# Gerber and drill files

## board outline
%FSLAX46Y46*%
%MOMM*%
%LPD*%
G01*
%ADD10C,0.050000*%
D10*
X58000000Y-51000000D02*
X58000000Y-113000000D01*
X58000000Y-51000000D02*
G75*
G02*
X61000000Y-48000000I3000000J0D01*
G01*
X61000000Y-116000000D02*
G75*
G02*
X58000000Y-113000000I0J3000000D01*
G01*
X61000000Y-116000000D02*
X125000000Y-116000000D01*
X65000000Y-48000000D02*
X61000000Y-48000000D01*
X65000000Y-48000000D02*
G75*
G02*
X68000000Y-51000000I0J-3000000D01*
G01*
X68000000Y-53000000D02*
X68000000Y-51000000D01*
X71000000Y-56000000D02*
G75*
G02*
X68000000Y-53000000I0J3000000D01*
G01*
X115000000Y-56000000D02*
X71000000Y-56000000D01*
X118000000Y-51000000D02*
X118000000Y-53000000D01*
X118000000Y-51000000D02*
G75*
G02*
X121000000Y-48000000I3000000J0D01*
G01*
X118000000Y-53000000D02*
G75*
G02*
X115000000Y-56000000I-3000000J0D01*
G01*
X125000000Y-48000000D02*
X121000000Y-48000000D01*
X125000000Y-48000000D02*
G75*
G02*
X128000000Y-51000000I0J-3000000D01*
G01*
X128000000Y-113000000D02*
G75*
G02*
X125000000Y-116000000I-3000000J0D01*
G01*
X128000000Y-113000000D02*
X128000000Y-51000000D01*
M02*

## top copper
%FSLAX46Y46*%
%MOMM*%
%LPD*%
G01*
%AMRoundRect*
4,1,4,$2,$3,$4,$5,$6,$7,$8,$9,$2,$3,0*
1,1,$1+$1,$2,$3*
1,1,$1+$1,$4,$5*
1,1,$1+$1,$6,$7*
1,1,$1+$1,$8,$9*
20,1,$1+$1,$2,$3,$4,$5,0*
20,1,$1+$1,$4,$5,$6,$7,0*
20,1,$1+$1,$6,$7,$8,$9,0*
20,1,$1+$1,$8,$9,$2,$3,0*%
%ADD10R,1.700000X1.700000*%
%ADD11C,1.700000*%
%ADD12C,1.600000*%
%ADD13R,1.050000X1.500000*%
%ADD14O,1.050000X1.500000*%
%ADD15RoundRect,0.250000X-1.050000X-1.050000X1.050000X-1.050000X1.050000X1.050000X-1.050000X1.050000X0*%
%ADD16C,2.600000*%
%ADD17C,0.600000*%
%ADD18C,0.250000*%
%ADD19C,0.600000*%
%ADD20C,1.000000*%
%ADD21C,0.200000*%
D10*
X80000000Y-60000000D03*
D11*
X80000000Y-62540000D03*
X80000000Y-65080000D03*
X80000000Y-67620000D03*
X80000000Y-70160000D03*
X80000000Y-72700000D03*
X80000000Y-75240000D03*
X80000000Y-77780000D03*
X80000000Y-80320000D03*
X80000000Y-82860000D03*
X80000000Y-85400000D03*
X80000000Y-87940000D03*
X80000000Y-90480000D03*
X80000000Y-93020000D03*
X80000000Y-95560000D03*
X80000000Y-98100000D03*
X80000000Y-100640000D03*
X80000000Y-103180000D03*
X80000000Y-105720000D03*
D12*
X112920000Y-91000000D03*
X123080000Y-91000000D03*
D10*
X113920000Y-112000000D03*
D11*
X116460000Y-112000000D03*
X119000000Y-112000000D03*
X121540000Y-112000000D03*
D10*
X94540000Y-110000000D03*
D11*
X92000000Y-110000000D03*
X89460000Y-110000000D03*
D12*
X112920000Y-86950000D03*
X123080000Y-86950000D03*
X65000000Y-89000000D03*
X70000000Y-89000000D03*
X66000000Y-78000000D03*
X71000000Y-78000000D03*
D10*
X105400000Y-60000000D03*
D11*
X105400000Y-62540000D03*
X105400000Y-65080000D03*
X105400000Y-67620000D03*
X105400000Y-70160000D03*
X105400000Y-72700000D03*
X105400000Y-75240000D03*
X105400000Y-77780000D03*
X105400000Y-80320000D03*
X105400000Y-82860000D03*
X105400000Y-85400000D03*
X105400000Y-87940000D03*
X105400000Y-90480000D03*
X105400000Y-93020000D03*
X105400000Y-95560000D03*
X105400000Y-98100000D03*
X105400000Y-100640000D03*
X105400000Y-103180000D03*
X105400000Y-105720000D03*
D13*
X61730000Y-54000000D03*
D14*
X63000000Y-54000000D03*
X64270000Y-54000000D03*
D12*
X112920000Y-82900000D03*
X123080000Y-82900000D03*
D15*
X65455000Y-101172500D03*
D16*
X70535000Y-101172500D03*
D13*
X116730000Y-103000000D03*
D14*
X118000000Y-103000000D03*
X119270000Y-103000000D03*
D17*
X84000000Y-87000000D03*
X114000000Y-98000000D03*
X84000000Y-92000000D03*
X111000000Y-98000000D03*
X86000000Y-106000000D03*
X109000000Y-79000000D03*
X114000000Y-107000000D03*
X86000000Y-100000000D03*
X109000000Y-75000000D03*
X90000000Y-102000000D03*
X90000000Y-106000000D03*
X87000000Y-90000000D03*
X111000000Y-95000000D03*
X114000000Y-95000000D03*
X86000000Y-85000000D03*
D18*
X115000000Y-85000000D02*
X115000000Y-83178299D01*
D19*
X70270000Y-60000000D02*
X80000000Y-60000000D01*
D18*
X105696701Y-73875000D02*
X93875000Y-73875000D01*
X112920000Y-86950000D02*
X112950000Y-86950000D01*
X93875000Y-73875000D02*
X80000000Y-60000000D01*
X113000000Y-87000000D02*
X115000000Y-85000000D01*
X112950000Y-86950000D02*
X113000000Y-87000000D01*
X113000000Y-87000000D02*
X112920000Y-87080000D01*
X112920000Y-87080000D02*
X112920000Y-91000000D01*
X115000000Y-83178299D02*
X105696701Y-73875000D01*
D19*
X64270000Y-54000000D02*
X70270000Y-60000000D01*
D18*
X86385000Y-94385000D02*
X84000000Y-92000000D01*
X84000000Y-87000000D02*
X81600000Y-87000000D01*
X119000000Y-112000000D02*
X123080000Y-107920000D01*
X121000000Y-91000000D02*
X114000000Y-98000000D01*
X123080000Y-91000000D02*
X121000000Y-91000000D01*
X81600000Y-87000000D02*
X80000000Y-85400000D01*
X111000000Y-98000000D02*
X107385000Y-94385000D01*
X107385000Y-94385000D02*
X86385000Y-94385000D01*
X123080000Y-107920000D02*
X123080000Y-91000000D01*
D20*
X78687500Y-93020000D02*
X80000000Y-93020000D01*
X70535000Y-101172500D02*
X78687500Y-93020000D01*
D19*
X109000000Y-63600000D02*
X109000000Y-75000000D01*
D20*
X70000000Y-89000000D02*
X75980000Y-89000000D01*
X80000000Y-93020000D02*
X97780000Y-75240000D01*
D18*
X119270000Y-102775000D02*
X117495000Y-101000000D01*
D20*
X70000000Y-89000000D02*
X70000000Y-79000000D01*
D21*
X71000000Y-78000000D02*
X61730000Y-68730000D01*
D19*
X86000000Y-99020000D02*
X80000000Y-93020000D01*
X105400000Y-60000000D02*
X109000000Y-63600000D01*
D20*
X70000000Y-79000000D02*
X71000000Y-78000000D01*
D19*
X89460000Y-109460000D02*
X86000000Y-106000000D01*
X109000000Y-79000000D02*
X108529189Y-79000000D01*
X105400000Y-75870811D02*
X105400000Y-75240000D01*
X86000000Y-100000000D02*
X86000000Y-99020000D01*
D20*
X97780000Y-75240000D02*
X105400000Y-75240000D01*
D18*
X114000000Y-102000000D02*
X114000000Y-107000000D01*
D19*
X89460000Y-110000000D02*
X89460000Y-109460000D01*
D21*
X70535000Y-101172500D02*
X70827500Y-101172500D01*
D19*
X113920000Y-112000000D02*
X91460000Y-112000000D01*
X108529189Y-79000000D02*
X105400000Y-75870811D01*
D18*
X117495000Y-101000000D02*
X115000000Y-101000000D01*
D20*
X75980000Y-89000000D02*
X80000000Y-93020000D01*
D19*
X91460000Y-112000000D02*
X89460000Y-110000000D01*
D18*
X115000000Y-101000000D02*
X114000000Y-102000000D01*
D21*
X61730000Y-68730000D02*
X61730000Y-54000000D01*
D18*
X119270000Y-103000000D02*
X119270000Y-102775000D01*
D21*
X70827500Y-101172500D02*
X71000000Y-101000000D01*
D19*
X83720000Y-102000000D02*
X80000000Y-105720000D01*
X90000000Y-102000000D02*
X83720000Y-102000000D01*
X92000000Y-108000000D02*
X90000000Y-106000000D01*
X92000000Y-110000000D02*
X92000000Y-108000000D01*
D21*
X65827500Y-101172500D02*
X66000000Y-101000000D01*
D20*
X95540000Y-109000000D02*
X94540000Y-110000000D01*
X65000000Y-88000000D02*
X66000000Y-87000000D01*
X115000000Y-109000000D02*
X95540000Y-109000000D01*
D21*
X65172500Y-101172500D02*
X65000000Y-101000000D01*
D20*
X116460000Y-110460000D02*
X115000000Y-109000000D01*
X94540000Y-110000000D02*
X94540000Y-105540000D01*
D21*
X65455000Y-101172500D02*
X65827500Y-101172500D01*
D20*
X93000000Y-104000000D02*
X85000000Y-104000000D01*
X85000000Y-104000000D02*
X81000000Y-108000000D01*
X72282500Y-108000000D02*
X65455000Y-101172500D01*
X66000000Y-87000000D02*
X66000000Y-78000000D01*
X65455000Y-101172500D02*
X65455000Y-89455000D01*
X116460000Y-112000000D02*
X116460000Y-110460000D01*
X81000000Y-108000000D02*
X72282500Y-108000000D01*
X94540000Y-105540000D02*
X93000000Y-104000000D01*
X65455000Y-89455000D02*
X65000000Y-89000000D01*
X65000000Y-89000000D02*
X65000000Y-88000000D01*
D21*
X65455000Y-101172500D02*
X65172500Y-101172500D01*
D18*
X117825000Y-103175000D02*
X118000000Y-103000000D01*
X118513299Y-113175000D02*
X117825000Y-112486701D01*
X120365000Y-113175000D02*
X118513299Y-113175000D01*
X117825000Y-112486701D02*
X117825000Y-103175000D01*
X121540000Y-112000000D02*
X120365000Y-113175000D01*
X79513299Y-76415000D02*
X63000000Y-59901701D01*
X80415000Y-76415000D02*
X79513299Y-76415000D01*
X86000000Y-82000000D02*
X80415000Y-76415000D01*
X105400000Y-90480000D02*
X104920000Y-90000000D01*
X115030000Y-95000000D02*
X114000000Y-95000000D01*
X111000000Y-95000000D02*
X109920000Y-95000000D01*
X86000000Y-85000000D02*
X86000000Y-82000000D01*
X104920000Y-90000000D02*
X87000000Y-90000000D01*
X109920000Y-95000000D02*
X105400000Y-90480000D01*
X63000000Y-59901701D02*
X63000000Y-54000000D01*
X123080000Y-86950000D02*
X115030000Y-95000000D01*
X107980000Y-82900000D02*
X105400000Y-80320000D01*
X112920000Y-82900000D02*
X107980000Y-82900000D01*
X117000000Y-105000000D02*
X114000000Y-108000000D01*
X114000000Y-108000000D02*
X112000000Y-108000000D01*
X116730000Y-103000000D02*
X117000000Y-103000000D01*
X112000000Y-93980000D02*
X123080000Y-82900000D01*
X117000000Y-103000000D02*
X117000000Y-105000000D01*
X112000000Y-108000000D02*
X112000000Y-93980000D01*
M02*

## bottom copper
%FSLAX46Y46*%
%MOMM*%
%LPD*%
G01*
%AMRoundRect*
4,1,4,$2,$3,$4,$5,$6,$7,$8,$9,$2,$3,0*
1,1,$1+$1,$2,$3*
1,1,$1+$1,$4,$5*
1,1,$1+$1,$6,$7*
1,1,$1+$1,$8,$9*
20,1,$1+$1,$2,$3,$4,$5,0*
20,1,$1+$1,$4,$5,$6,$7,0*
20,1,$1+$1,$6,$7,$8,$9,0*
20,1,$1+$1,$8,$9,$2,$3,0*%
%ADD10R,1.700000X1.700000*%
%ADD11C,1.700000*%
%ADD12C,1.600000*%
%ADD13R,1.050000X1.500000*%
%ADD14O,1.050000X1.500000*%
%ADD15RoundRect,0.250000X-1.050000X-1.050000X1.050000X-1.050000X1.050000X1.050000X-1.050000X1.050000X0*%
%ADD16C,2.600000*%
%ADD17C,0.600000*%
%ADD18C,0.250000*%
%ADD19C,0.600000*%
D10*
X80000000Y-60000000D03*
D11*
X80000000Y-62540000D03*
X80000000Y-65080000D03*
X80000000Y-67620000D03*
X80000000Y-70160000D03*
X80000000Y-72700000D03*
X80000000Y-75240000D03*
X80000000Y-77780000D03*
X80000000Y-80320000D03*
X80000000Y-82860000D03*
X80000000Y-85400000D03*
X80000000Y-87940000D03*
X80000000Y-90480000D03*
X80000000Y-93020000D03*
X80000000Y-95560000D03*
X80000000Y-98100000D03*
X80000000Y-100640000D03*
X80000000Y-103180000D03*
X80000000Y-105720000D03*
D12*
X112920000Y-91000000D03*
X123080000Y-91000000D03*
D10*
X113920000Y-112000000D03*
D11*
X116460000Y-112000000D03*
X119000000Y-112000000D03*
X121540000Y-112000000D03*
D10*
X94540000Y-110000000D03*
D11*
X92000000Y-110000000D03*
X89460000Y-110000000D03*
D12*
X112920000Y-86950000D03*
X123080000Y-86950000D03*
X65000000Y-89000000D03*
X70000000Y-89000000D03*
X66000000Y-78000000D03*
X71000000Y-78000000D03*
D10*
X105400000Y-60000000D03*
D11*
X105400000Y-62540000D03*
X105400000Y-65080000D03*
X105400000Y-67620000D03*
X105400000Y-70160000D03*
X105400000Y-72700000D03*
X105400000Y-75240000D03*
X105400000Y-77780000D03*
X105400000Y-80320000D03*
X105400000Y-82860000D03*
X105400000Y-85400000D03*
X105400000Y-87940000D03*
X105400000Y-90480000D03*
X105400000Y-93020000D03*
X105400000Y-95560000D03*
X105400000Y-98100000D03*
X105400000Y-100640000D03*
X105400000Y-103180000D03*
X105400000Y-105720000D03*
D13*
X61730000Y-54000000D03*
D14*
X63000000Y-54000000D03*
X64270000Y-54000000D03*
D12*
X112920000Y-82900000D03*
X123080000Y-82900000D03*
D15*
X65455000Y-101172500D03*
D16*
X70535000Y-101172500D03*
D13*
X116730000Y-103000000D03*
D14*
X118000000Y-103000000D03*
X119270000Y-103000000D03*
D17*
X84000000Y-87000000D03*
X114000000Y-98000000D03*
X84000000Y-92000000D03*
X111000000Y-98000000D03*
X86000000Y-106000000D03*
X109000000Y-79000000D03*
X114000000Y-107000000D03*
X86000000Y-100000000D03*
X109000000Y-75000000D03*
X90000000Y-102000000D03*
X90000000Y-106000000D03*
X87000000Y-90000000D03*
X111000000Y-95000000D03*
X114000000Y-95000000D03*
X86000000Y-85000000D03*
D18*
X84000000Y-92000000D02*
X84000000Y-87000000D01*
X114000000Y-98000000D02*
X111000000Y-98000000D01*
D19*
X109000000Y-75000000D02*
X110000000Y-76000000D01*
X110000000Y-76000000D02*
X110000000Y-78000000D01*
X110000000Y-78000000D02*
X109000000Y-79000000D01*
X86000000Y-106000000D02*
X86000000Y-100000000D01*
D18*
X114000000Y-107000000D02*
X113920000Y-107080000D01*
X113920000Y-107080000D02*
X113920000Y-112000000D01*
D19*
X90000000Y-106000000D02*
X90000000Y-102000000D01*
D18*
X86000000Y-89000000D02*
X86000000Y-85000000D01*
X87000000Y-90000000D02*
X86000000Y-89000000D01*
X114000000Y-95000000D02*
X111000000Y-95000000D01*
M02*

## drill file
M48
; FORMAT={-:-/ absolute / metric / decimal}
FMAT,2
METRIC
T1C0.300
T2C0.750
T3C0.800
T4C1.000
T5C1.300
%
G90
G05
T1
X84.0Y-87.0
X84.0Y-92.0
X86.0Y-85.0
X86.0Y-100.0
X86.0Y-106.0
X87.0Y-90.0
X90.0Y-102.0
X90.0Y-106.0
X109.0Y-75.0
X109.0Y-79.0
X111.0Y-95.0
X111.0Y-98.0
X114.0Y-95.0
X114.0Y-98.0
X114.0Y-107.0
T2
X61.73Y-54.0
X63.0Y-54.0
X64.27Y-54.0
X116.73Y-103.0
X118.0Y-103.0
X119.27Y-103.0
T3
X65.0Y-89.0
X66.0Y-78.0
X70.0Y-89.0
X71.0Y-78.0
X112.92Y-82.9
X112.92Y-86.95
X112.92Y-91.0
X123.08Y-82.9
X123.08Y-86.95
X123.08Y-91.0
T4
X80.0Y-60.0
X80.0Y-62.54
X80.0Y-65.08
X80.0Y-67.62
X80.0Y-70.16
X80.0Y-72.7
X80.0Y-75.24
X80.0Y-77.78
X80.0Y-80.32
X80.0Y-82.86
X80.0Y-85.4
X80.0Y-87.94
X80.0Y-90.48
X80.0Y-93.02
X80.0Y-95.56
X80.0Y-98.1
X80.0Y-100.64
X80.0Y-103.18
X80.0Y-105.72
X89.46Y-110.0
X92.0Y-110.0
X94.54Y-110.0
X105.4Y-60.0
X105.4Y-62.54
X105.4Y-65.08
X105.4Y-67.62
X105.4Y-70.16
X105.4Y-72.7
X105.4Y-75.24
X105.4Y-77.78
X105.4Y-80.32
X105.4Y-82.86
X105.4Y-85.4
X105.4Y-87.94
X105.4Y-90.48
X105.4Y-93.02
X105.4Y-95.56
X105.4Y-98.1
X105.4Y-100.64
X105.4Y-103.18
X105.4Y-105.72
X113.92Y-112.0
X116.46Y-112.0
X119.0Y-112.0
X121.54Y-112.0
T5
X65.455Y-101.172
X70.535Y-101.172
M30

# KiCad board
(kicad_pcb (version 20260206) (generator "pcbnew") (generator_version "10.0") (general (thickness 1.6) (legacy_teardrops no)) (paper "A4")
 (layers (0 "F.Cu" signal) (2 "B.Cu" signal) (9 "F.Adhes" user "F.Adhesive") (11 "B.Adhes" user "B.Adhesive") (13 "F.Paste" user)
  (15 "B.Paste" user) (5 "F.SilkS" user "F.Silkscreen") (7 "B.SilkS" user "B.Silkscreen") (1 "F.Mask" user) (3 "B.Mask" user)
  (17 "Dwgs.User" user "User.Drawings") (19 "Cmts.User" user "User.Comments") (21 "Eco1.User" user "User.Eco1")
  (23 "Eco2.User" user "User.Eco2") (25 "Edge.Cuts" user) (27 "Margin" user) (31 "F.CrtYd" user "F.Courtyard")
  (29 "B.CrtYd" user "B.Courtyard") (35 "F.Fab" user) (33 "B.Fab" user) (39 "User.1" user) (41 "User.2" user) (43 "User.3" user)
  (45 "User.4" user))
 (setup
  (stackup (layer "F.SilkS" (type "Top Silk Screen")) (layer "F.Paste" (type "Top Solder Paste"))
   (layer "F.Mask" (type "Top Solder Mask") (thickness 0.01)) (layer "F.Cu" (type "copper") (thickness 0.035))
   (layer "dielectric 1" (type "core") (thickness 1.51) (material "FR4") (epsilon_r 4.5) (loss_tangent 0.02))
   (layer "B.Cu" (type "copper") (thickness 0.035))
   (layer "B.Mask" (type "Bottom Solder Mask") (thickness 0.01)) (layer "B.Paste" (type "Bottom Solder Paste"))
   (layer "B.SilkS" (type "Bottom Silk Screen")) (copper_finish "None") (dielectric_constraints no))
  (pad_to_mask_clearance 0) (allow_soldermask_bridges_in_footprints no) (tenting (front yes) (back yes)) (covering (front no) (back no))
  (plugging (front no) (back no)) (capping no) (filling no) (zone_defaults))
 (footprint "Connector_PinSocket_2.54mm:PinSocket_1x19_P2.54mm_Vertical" (layer "F.Cu") (at 80 60)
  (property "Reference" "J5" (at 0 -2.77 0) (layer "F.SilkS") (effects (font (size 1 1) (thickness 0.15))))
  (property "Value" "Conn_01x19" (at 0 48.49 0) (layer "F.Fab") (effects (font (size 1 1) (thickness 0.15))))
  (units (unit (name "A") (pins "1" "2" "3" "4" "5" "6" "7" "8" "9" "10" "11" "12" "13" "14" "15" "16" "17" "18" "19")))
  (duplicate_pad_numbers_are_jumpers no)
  (pad "1" thru_hole rect (at 0 0) (size 1.7 1.7) (drill 1) (layers "*.Cu" "*.Mask") (remove_unused_layers no) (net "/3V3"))
  (pad "2" thru_hole circle (at 0 2.54) (size 1.7 1.7) (drill 1) (layers "*.Cu" "*.Mask") (remove_unused_layers no)
   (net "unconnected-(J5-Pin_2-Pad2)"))
  (pad "3" thru_hole circle (at 0 5.08) (size 1.7 1.7) (drill 1) (layers "*.Cu" "*.Mask") (remove_unused_layers no)
   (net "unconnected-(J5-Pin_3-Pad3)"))
  (pad "4" thru_hole circle (at 0 7.62) (size 1.7 1.7) (drill 1) (layers "*.Cu" "*.Mask") (remove_unused_layers no)
   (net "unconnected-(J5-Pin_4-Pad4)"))
  (pad "5" thru_hole circle (at 0 10.16) (size 1.7 1.7) (drill 1) (layers "*.Cu" "*.Mask") (remove_unused_layers no)
   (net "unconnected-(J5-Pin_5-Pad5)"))
  (pad "6" thru_hole circle (at 0 12.7) (size 1.7 1.7) (drill 1) (layers "*.Cu" "*.Mask") (remove_unused_layers no)
   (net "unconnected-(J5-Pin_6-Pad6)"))
  (pad "7" thru_hole circle (at 0 15.24) (size 1.7 1.7) (drill 1) (layers "*.Cu" "*.Mask") (remove_unused_layers no)
   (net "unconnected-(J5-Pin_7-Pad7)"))
  (pad "8" thru_hole circle (at 0 17.78) (size 1.7 1.7) (drill 1) (layers "*.Cu" "*.Mask") (remove_unused_layers no)
   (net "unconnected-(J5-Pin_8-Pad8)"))
  (pad "9" thru_hole circle (at 0 20.32) (size 1.7 1.7) (drill 1) (layers "*.Cu" "*.Mask") (remove_unused_layers no)
   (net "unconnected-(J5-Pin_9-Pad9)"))
  (pad "10" thru_hole circle (at 0 22.86) (size 1.7 1.7) (drill 1) (layers "*.Cu" "*.Mask") (remove_unused_layers no)
   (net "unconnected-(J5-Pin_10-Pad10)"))
  (pad "11" thru_hole circle (at 0 25.4) (size 1.7 1.7) (drill 1) (layers "*.Cu" "*.Mask") (remove_unused_layers no) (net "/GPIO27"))
  (pad "12" thru_hole circle (at 0 27.94) (size 1.7 1.7) (drill 1) (layers "*.Cu" "*.Mask") (remove_unused_layers no)
   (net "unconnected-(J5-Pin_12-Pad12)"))
  (pad "13" thru_hole circle (at 0 30.48) (size 1.7 1.7) (drill 1) (layers "*.Cu" "*.Mask") (remove_unused_layers no)
   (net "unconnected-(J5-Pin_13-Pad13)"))
  (pad "14" thru_hole circle (at 0 33.02) (size 1.7 1.7) (drill 1) (layers "*.Cu" "*.Mask") (remove_unused_layers no) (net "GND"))
  (pad "15" thru_hole circle (at 0 35.56) (size 1.7 1.7) (drill 1) (layers "*.Cu" "*.Mask") (remove_unused_layers no)
   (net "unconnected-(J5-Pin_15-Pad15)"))
  (pad "16" thru_hole circle (at 0 38.1) (size 1.7 1.7) (drill 1) (layers "*.Cu" "*.Mask") (remove_unused_layers no)
   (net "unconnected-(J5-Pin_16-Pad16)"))
  (pad "17" thru_hole circle (at 0 40.64) (size 1.7 1.7) (drill 1) (layers "*.Cu" "*.Mask") (remove_unused_layers no)
   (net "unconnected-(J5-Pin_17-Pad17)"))
  (pad "18" thru_hole circle (at 0 43.18) (size 1.7 1.7) (drill 1) (layers "*.Cu" "*.Mask") (remove_unused_layers no)
   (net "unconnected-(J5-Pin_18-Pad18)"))
  (pad "19" thru_hole circle (at 0 45.72) (size 1.7 1.7) (drill 1) (layers "*.Cu" "*.Mask") (remove_unused_layers no) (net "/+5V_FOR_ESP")))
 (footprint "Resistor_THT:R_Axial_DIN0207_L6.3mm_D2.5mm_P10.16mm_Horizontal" (layer "F.Cu") (at 112.92 91)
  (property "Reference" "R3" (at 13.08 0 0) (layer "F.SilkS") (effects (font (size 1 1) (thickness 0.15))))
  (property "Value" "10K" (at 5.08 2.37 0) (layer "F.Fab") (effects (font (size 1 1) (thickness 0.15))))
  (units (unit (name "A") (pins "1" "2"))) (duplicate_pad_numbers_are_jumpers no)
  (pad "1" thru_hole circle (at 0 0) (size 1.6 1.6) (drill 0.8) (layers "*.Cu" "*.Mask") (remove_unused_layers no) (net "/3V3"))
  (pad "2" thru_hole circle (at 10.16 0) (size 1.6 1.6) (drill 0.8) (layers "*.Cu" "*.Mask") (remove_unused_layers no) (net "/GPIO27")))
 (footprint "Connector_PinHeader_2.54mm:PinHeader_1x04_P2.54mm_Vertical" (layer "F.Cu") (at 113.92 112 90)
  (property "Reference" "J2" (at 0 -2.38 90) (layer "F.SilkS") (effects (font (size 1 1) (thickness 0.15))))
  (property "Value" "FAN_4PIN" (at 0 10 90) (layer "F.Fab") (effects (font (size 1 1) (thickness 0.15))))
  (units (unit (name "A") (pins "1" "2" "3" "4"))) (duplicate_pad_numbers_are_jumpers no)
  (pad "1" thru_hole rect (at 0 0 90) (size 1.7 1.7) (drill 1) (layers "*.Cu" "*.Mask") (remove_unused_layers no) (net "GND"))
  (pad "2" thru_hole circle (at 0 2.54 90) (size 1.7 1.7) (drill 1) (layers "*.Cu" "*.Mask") (remove_unused_layers no) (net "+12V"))
  (pad "3" thru_hole circle (at 0 5.08 90) (size 1.7 1.7) (drill 1) (layers "*.Cu" "*.Mask") (remove_unused_layers no) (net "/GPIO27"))
  (pad "4" thru_hole circle (at 0 7.62 90) (size 1.7 1.7) (drill 1) (layers "*.Cu" "*.Mask") (remove_unused_layers no) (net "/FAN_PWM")))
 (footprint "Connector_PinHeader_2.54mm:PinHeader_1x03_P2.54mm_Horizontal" (layer "F.Cu") (at 94.54 110 -90)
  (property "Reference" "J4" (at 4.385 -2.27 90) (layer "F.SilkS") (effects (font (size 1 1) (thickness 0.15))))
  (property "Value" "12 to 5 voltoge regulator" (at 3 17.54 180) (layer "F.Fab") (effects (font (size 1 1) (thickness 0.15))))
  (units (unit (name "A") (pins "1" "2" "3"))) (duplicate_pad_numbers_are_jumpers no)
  (pad "1" thru_hole rect (at 0 0 270) (size 1.7 1.7) (drill 1) (layers "*.Cu" "*.Mask") (remove_unused_layers no) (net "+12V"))
  (pad "2" thru_hole circle (at 0 2.54 270) (size 1.7 1.7) (drill 1) (layers "*.Cu" "*.Mask") (remove_unused_layers no) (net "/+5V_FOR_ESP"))
  (pad "3" thru_hole circle (at 0 5.08 270) (size 1.7 1.7) (drill 1) (layers "*.Cu" "*.Mask") (remove_unused_layers no) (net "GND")))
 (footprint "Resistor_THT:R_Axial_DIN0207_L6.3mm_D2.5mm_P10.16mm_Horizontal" (layer "F.Cu") (at 112.92 86.95)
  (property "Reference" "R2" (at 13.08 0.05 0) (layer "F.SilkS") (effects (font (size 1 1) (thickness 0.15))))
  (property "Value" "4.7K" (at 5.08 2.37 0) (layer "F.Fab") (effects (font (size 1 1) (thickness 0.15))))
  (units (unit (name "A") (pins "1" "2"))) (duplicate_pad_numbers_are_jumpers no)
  (pad "1" thru_hole circle (at 0 0) (size 1.6 1.6) (drill 0.8) (layers "*.Cu" "*.Mask") (remove_unused_layers no) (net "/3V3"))
  (pad "2" thru_hole circle (at 10.16 0) (size 1.6 1.6) (drill 0.8) (layers "*.Cu" "*.Mask") (remove_unused_layers no) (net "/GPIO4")))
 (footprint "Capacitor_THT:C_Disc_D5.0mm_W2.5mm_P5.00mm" (layer "F.Cu") (at 65 89)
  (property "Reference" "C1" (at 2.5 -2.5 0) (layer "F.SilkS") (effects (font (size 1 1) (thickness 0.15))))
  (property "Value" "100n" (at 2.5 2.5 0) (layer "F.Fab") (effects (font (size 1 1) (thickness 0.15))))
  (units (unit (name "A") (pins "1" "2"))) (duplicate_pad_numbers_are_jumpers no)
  (pad "1" thru_hole circle (at 0 0) (size 1.6 1.6) (drill 0.8) (layers "*.Cu" "*.Mask") (remove_unused_layers no) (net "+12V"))
  (pad "2" thru_hole circle (at 5 0) (size 1.6 1.6) (drill 0.8) (layers "*.Cu" "*.Mask") (remove_unused_layers no) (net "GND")))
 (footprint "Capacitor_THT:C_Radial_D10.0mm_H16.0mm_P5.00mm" (layer "F.Cu") (at 66 78)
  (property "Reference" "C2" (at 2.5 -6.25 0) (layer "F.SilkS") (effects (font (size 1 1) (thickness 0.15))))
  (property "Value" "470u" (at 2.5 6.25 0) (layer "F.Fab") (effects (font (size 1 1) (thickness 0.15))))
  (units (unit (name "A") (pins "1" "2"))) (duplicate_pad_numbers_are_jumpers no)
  (pad "1" thru_hole circle (at 0 0) (size 1.6 1.6) (drill 0.8) (layers "*.Cu" "*.Mask") (remove_unused_layers no) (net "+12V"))
  (pad "2" thru_hole circle (at 5 0) (size 1.6 1.6) (drill 0.8) (layers "*.Cu" "*.Mask") (remove_unused_layers no) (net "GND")))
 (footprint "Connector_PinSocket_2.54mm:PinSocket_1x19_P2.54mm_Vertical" (layer "F.Cu") (at 105.4 60)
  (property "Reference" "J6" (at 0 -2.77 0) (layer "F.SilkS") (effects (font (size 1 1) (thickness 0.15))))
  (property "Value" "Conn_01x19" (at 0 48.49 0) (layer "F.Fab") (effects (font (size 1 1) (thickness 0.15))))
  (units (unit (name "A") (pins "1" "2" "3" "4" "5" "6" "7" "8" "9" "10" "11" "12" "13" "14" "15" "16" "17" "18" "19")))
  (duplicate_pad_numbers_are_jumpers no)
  (pad "1" thru_hole rect (at 0 0) (size 1.7 1.7) (drill 1) (layers "*.Cu" "*.Mask") (remove_unused_layers no) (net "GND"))
  (pad "2" thru_hole circle (at 0 2.54) (size 1.7 1.7) (drill 1) (layers "*.Cu" "*.Mask") (remove_unused_layers no)
   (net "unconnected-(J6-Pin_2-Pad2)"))
  (pad "3" thru_hole circle (at 0 5.08) (size 1.7 1.7) (drill 1) (layers "*.Cu" "*.Mask") (remove_unused_layers no)
   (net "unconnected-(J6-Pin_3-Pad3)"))
  (pad "4" thru_hole circle (at 0 7.62) (size 1.7 1.7) (drill 1) (layers "*.Cu" "*.Mask") (remove_unused_layers no)
   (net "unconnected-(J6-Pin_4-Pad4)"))
  (pad "5" thru_hole circle (at 0 10.16) (size 1.7 1.7) (drill 1) (layers "*.Cu" "*.Mask") (remove_unused_layers no)
   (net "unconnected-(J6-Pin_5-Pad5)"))
  (pad "6" thru_hole circle (at 0 12.7) (size 1.7 1.7) (drill 1) (layers "*.Cu" "*.Mask") (remove_unused_layers no)
   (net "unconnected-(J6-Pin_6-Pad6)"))
  (pad "7" thru_hole circle (at 0 15.24) (size 1.7 1.7) (drill 1) (layers "*.Cu" "*.Mask") (remove_unused_layers no) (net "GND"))
  (pad "8" thru_hole circle (at 0 17.78) (size 1.7 1.7) (drill 1) (layers "*.Cu" "*.Mask") (remove_unused_layers no)
   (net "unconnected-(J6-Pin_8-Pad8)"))
  (pad "9" thru_hole circle (at 0 20.32) (size 1.7 1.7) (drill 1) (layers "*.Cu" "*.Mask") (remove_unused_layers no) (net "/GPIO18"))
  (pad "10" thru_hole circle (at 0 22.86) (size 1.7 1.7) (drill 1) (layers "*.Cu" "*.Mask") (remove_unused_layers no)
   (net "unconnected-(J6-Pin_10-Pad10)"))
  (pad "11" thru_hole circle (at 0 25.4) (size 1.7 1.7) (drill 1) (layers "*.Cu" "*.Mask") (remove_unused_layers no)
   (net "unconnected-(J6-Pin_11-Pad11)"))
  (pad "12" thru_hole circle (at 0 27.94) (size 1.7 1.7) (drill 1) (layers "*.Cu" "*.Mask") (remove_unused_layers no)
   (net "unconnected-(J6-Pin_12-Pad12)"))
  (pad "13" thru_hole circle (at 0 30.48) (size 1.7 1.7) (drill 1) (layers "*.Cu" "*.Mask") (remove_unused_layers no) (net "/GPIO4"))
  (pad "14" thru_hole circle (at 0 33.02) (size 1.7 1.7) (drill 1) (layers "*.Cu" "*.Mask") (remove_unused_layers no)
   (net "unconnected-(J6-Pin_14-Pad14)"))
  (pad "15" thru_hole circle (at 0 35.56) (size 1.7 1.7) (drill 1) (layers "*.Cu" "*.Mask") (remove_unused_layers no)
   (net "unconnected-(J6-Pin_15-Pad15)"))
  (pad "16" thru_hole circle (at 0 38.1) (size 1.7 1.7) (drill 1) (layers "*.Cu" "*.Mask") (remove_unused_layers no)
   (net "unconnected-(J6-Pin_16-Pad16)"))
  (pad "17" thru_hole circle (at 0 40.64) (size 1.7 1.7) (drill 1) (layers "*.Cu" "*.Mask") (remove_unused_layers no)
   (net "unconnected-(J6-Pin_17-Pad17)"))
  (pad "18" thru_hole circle (at 0 43.18) (size 1.7 1.7) (drill 1) (layers "*.Cu" "*.Mask") (remove_unused_layers no)
   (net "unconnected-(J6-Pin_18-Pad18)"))
  (pad "19" thru_hole circle (at 0 45.72) (size 1.7 1.7) (drill 1) (layers "*.Cu" "*.Mask") (remove_unused_layers no)
   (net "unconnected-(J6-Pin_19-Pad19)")))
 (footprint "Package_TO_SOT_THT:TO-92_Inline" (layer "F.Cu") (at 61.73 54)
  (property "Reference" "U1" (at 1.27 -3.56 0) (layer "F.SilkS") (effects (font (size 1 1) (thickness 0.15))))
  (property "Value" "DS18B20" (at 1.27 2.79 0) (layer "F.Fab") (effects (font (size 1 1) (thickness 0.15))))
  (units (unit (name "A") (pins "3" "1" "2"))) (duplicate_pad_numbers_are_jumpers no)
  (pad "1" thru_hole rect (at 0 0) (size 1.05 1.5) (drill 0.75) (layers "*.Cu" "*.Mask") (remove_unused_layers no) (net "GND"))
  (pad "2" thru_hole oval (at 1.27 0) (size 1.05 1.5) (drill 0.75) (layers "*.Cu" "*.Mask") (remove_unused_layers no) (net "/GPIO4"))
  (pad "3" thru_hole oval (at 2.54 0) (size 1.05 1.5) (drill 0.75) (layers "*.Cu" "*.Mask") (remove_unused_layers no) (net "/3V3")))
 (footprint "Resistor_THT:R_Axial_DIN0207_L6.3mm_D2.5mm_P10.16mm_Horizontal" (layer "F.Cu") (at 112.92 82.9)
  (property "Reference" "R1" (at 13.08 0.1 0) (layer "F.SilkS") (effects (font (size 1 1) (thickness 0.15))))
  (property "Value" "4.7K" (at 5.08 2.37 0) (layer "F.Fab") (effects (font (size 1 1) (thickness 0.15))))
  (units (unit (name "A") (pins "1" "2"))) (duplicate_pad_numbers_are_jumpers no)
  (pad "1" thru_hole circle (at 0 0) (size 1.6 1.6) (drill 0.8) (layers "*.Cu" "*.Mask") (remove_unused_layers no) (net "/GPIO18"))
  (pad "2" thru_hole circle (at 10.16 0) (size 1.6 1.6) (drill 0.8) (layers "*.Cu" "*.Mask") (remove_unused_layers no) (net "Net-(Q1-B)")))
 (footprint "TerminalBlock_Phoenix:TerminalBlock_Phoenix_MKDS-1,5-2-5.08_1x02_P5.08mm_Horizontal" (layer "F.Cu") (at 65.455 101.1725)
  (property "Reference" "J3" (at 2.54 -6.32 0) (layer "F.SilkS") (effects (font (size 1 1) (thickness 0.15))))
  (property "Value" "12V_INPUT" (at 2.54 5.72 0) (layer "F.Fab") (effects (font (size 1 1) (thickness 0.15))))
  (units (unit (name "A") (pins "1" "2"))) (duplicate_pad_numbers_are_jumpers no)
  (pad "1" thru_hole roundrect (at 0 0) (size 2.6 2.6) (drill 1.3) (layers "*.Cu" "*.Mask") (remove_unused_layers no)
   (roundrect_rratio 0.096154) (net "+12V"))
  (pad "2" thru_hole circle (at 5.08 0) (size 2.6 2.6) (drill 1.3) (layers "*.Cu" "*.Mask") (remove_unused_layers no) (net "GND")))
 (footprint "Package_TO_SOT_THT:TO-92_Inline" (layer "F.Cu") (at 116.73 103)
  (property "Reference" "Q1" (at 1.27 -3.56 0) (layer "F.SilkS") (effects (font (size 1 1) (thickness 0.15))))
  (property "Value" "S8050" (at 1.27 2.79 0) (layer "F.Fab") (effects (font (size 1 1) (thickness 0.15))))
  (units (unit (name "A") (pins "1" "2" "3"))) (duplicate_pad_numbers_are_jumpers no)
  (pad "1" thru_hole rect (at 0 0) (size 1.05 1.5) (drill 0.75) (layers "*.Cu" "*.Mask") (remove_unused_layers no) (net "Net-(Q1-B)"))
  (pad "2" thru_hole oval (at 1.27 0) (size 1.05 1.5) (drill 0.75) (layers "*.Cu" "*.Mask") (remove_unused_layers no) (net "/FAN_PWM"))
  (pad "3" thru_hole oval (at 2.54 0) (size 1.05 1.5) (drill 0.75) (layers "*.Cu" "*.Mask") (remove_unused_layers no) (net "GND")))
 (gr_line (start 58 51) (end 58 113) (stroke (width 0.05) (type default)) (layer "Edge.Cuts"))
 (gr_arc (start 58 51) (mid 58.87868 48.87868) (end 61 48) (stroke (width 0.05) (type default)) (layer "Edge.Cuts"))
 (gr_arc (start 61 116) (mid 58.87868 115.12132) (end 58 113) (stroke (width 0.05) (type default)) (layer "Edge.Cuts"))
 (gr_line (start 61 116) (end 125 116) (stroke (width 0.05) (type default)) (layer "Edge.Cuts"))
 (gr_line (start 65 48) (end 61 48) (stroke (width 0.05) (type default)) (layer "Edge.Cuts"))
 (gr_arc (start 65 48) (mid 67.12132 48.87868) (end 68 51) (stroke (width 0.05) (type default)) (layer "Edge.Cuts"))
 (gr_line (start 68 53) (end 68 51) (stroke (width 0.05) (type default)) (layer "Edge.Cuts"))
 (gr_arc (start 71 56) (mid 68.87868 55.12132) (end 68 53) (stroke (width 0.05) (type default)) (layer "Edge.Cuts"))
 (gr_line (start 115 56) (end 71 56) (stroke (width 0.05) (type default)) (layer "Edge.Cuts"))
 (gr_line (start 118 51) (end 118 53) (stroke (width 0.05) (type default)) (layer "Edge.Cuts"))
 (gr_arc (start 118 51) (mid 118.87868 48.87868) (end 121 48) (stroke (width 0.05) (type default)) (layer "Edge.Cuts"))
 (gr_arc (start 118 53) (mid 117.12132 55.12132) (end 115 56) (stroke (width 0.05) (type default)) (layer "Edge.Cuts"))
 (gr_line (start 125 48) (end 121 48) (stroke (width 0.05) (type default)) (layer "Edge.Cuts"))
 (gr_arc (start 125 48) (mid 127.12132 48.87868) (end 128 51) (stroke (width 0.05) (type default)) (layer "Edge.Cuts"))
 (gr_arc (start 128 113) (mid 127.12132 115.12132) (end 125 116) (stroke (width 0.05) (type default)) (layer "Edge.Cuts"))
 (gr_line (start 128 113) (end 128 51) (stroke (width 0.05) (type default)) (layer "Edge.Cuts"))
 (segment (start 115 85) (end 115 83.178299) (width 0.25) (layer "F.Cu") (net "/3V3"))
 (segment (start 70.27 60) (end 80 60) (width 0.6) (layer "F.Cu") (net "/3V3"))
 (segment (start 105.696701 73.875) (end 93.875 73.875) (width 0.25) (layer "F.Cu") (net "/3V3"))
 (segment (start 112.92 86.95) (end 112.95 86.95) (width 0.25) (layer "F.Cu") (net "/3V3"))
 (segment (start 93.875 73.875) (end 80 60) (width 0.25) (layer "F.Cu") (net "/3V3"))
 (segment (start 113 87) (end 115 85) (width 0.25) (layer "F.Cu") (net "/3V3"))
 (segment (start 112.95 86.95) (end 113 87) (width 0.25) (layer "F.Cu") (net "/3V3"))
 (segment (start 113 87) (end 112.92 87.08) (width 0.25) (layer "F.Cu") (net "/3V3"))
 (segment (start 112.92 87.08) (end 112.92 91) (width 0.25) (layer "F.Cu") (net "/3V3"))
 (segment (start 115 83.178299) (end 105.696701 73.875) (width 0.25) (layer "F.Cu") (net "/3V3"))
 (segment (start 64.27 54) (end 70.27 60) (width 0.6) (layer "F.Cu") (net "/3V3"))
 (segment (start 86.385 94.385) (end 84 92) (width 0.25) (layer "F.Cu") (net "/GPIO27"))
 (segment (start 84 87) (end 81.6 87) (width 0.25) (layer "F.Cu") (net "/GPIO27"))
 (segment (start 119 112) (end 123.08 107.92) (width 0.25) (layer "F.Cu") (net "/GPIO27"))
 (segment (start 121 91) (end 114 98) (width 0.25) (layer "F.Cu") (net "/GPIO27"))
 (segment (start 123.08 91) (end 121 91) (width 0.25) (layer "F.Cu") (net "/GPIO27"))
 (segment (start 81.6 87) (end 80 85.4) (width 0.25) (layer "F.Cu") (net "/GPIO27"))
 (segment (start 111 98) (end 107.385 94.385) (width 0.25) (layer "F.Cu") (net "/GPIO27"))
 (segment (start 107.385 94.385) (end 86.385 94.385) (width 0.25) (layer "F.Cu") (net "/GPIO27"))
 (segment (start 123.08 107.92) (end 123.08 91) (width 0.25) (layer "F.Cu") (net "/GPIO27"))
 (via (at 84 87) (size 0.6) (drill 0.3) (layers "F.Cu" "B.Cu") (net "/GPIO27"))
 (via (at 114 98) (size 0.6) (drill 0.3) (layers "F.Cu" "B.Cu") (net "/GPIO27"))
 (via (at 84 92) (size 0.6) (drill 0.3) (layers "F.Cu" "B.Cu") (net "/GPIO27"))
 (via (at 111 98) (size 0.6) (drill 0.3) (layers "F.Cu" "B.Cu") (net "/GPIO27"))
 (segment (start 84 92) (end 84 87) (width 0.25) (layer "B.Cu") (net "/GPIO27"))
 (segment (start 114 98) (end 111 98) (width 0.25) (layer "B.Cu") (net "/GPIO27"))
 (segment (start 78.6875 93.02) (end 80 93.02) (width 1) (layer "F.Cu") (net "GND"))
 (segment (start 70.535 101.1725) (end 78.6875 93.02) (width 1) (layer "F.Cu") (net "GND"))
 (segment (start 109 63.6) (end 109 75) (width 0.6) (layer "F.Cu") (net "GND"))
 (segment (start 70 89) (end 75.98 89) (width 1) (layer "F.Cu") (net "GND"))
 (segment (start 80 93.02) (end 97.78 75.24) (width 1) (layer "F.Cu") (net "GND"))
 (segment (start 119.27 102.775) (end 117.495 101) (width 0.25) (layer "F.Cu") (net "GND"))
 (segment (start 70 89) (end 70 79) (width 1) (layer "F.Cu") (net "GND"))
 (segment (start 71 78) (end 61.73 68.73) (width 0.2) (layer "F.Cu") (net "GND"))
 (segment (start 86 99.02) (end 80 93.02) (width 0.6) (layer "F.Cu") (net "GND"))
 (segment (start 105.4 60) (end 109 63.6) (width 0.6) (layer "F.Cu") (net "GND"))
 (segment (start 70 79) (end 71 78) (width 1) (layer "F.Cu") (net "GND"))
 (segment (start 89.46 109.46) (end 86 106) (width 0.6) (layer "F.Cu") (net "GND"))
 (segment (start 109 79) (end 108.529189 79) (width 0.6) (layer "F.Cu") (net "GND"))
 (segment (start 105.4 75.870811) (end 105.4 75.24) (width 0.6) (layer "F.Cu") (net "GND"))
 (segment (start 86 100) (end 86 99.02) (width 0.6) (layer "F.Cu") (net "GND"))
 (segment (start 97.78 75.24) (end 105.4 75.24) (width 1) (layer "F.Cu") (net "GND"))
 (segment (start 114 102) (end 114 107) (width 0.25) (layer "F.Cu") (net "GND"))
 (segment (start 89.46 110) (end 89.46 109.46) (width 0.6) (layer "F.Cu") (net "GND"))
 (segment (start 70.535 101.1725) (end 70.8275 101.1725) (width 0.2) (layer "F.Cu") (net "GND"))
 (segment (start 113.92 112) (end 91.46 112) (width 0.6) (layer "F.Cu") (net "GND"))
 (segment (start 108.529189 79) (end 105.4 75.870811) (width 0.6) (layer "F.Cu") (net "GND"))
 (segment (start 117.495 101) (end 115 101) (width 0.25) (layer "F.Cu") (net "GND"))
 (segment (start 75.98 89) (end 80 93.02) (width 1) (layer "F.Cu") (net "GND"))
 (segment (start 91.46 112) (end 89.46 110) (width 0.6) (layer "F.Cu") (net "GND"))
 (segment (start 115 101) (end 114 102) (width 0.25) (layer "F.Cu") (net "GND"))
 (segment (start 61.73 68.73) (end 61.73 54) (width 0.2) (layer "F.Cu") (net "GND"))
 (segment (start 119.27 103) (end 119.27 102.775) (width 0.25) (layer "F.Cu") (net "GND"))
 (segment (start 70.8275 101.1725) (end 71 101) (width 0.2) (layer "F.Cu") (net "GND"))
 (via (at 86 106) (size 0.6) (drill 0.3) (layers "F.Cu" "B.Cu") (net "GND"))
 (via (at 109 79) (size 0.6) (drill 0.3) (layers "F.Cu" "B.Cu") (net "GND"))
 (via (at 114 107) (size 0.6) (drill 0.3) (layers "F.Cu" "B.Cu") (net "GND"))
 (via (at 86 100) (size 0.6) (drill 0.3) (layers "F.Cu" "B.Cu") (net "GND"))
 (via (at 109 75) (size 0.6) (drill 0.3) (layers "F.Cu" "B.Cu") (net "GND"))
 (segment (start 109 75) (end 110 76) (width 0.6) (layer "B.Cu") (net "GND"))
 (segment (start 110 76) (end 110 78) (width 0.6) (layer "B.Cu") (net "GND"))
 (segment (start 110 78) (end 109 79) (width 0.6) (layer "B.Cu") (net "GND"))
 (segment (start 86 106) (end 86 100) (width 0.6) (layer "B.Cu") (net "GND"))
 (segment (start 114 107) (end 113.92 107.08) (width 0.25) (layer "B.Cu") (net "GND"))
 (segment (start 113.92 107.08) (end 113.92 112) (width 0.25) (layer "B.Cu") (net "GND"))
 (segment (start 83.72 102) (end 80 105.72) (width 0.6) (layer "F.Cu") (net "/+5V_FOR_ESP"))
 (segment (start 90 102) (end 83.72 102) (width 0.6) (layer "F.Cu") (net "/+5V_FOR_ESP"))
 (segment (start 92 108) (end 90 106) (width 0.6) (layer "F.Cu") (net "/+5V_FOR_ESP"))
 (segment (start 92 110) (end 92 108) (width 0.6) (layer "F.Cu") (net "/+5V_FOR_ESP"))
 (via (at 90 102) (size 0.6) (drill 0.3) (layers "F.Cu" "B.Cu") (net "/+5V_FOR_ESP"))
 (via (at 90 106) (size 0.6) (drill 0.3) (layers "F.Cu" "B.Cu") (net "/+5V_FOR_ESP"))
 (segment (start 90 106) (end 90 102) (width 0.6) (layer "B.Cu") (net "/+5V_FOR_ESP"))
 (segment (start 65.8275 101.1725) (end 66 101) (width 0.2) (layer "F.Cu") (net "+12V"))
 (segment (start 95.54 109) (end 94.54 110) (width 1) (layer "F.Cu") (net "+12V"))
 (segment (start 65 88) (end 66 87) (width 1) (layer "F.Cu") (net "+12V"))
 (segment (start 115 109) (end 95.54 109) (width 1) (layer "F.Cu") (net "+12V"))
 (segment (start 65.1725 101.1725) (end 65 101) (width 0.2) (layer "F.Cu") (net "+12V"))
 (segment (start 116.46 110.46) (end 115 109) (width 1) (layer "F.Cu") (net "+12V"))
 (segment (start 94.54 110) (end 94.54 105.54) (width 1) (layer "F.Cu") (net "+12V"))
 (segment (start 65.455 101.1725) (end 65.8275 101.1725) (width 0.2) (layer "F.Cu") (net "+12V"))
 (segment (start 93 104) (end 85 104) (width 1) (layer "F.Cu") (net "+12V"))
 (segment (start 85 104) (end 81 108) (width 1) (layer "F.Cu") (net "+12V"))
 (segment (start 72.2825 108) (end 65.455 101.1725) (width 1) (layer "F.Cu") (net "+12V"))
 (segment (start 66 87) (end 66 78) (width 1) (layer "F.Cu") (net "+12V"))
 (segment (start 65.455 101.1725) (end 65.455 89.455) (width 1) (layer "F.Cu") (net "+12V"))
 (segment (start 116.46 112) (end 116.46 110.46) (width 1) (layer "F.Cu") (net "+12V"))
 (segment (start 81 108) (end 72.2825 108) (width 1) (layer "F.Cu") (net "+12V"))
 (segment (start 94.54 105.54) (end 93 104) (width 1) (layer "F.Cu") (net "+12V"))
 (segment (start 65.455 89.455) (end 65 89) (width 1) (layer "F.Cu") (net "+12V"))
 (segment (start 65 89) (end 65 88) (width 1) (layer "F.Cu") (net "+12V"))
 (segment (start 65.455 101.1725) (end 65.1725 101.1725) (width 0.2) (layer "F.Cu") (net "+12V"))
 (segment (start 117.825 103.175) (end 118 103) (width 0.25) (layer "F.Cu") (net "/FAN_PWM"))
 (segment (start 118.513299 113.175) (end 117.825 112.486701) (width 0.25) (layer "F.Cu") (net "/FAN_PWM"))
 (segment (start 120.365 113.175) (end 118.513299 113.175) (width 0.25) (layer "F.Cu") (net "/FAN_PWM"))
 (segment (start 117.825 112.486701) (end 117.825 103.175) (width 0.25) (layer "F.Cu") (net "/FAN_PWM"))
 (segment (start 121.54 112) (end 120.365 113.175) (width 0.25) (layer "F.Cu") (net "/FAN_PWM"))
 (segment (start 79.513299 76.415) (end 63 59.901701) (width 0.25) (layer "F.Cu") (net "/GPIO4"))
 (segment (start 80.415 76.415) (end 79.513299 76.415) (width 0.25) (layer "F.Cu") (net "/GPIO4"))
 (segment (start 86 82) (end 80.415 76.415) (width 0.25) (layer "F.Cu") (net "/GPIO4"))
 (segment (start 105.4 90.48) (end 104.92 90) (width 0.25) (layer "F.Cu") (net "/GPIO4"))
 (segment (start 115.03 95) (end 114 95) (width 0.25) (layer "F.Cu") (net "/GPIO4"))
 (segment (start 111 95) (end 109.92 95) (width 0.25) (layer "F.Cu") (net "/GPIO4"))
 (segment (start 86 85) (end 86 82) (width 0.25) (layer "F.Cu") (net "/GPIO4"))
 (segment (start 104.92 90) (end 87 90) (width 0.25) (layer "F.Cu") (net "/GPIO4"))
 (segment (start 109.92 95) (end 105.4 90.48) (width 0.25) (layer "F.Cu") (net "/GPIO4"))
 (segment (start 63 59.901701) (end 63 54) (width 0.25) (layer "F.Cu") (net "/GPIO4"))
 (segment (start 123.08 86.95) (end 115.03 95) (width 0.25) (layer "F.Cu") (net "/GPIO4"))
 (via (at 87 90) (size 0.6) (drill 0.3) (layers "F.Cu" "B.Cu") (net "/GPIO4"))
 (via (at 111 95) (size 0.6) (drill 0.3) (layers "F.Cu" "B.Cu") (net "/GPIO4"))
 (via (at 114 95) (size 0.6) (drill 0.3) (layers "F.Cu" "B.Cu") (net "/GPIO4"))
 (via (at 86 85) (size 0.6) (drill 0.3) (layers "F.Cu" "B.Cu") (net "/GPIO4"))
 (segment (start 86 89) (end 86 85) (width 0.25) (layer "B.Cu") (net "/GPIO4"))
 (segment (start 87 90) (end 86 89) (width 0.25) (layer "B.Cu") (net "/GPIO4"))
 (segment (start 114 95) (end 111 95) (width 0.25) (layer "B.Cu") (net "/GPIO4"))
 (segment (start 107.98 82.9) (end 105.4 80.32) (width 0.25) (layer "F.Cu") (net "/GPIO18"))
 (segment (start 112.92 82.9) (end 107.98 82.9) (width 0.25) (layer "F.Cu") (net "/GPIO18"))
 (segment (start 117 105) (end 114 108) (width 0.25) (layer "F.Cu") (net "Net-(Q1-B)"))
 (segment (start 114 108) (end 112 108) (width 0.25) (layer "F.Cu") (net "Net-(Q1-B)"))
 (segment (start 116.73 103) (end 117 103) (width 0.25) (layer "F.Cu") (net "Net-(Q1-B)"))
 (segment (start 112 93.98) (end 123.08 82.9) (width 0.25) (layer "F.Cu") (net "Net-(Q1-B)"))
 (segment (start 117 103) (end 117 105) (width 0.25) (layer "F.Cu") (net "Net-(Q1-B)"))
 (segment (start 112 108) (end 112 93.98) (width 0.25) (layer "F.Cu") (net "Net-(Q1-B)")))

